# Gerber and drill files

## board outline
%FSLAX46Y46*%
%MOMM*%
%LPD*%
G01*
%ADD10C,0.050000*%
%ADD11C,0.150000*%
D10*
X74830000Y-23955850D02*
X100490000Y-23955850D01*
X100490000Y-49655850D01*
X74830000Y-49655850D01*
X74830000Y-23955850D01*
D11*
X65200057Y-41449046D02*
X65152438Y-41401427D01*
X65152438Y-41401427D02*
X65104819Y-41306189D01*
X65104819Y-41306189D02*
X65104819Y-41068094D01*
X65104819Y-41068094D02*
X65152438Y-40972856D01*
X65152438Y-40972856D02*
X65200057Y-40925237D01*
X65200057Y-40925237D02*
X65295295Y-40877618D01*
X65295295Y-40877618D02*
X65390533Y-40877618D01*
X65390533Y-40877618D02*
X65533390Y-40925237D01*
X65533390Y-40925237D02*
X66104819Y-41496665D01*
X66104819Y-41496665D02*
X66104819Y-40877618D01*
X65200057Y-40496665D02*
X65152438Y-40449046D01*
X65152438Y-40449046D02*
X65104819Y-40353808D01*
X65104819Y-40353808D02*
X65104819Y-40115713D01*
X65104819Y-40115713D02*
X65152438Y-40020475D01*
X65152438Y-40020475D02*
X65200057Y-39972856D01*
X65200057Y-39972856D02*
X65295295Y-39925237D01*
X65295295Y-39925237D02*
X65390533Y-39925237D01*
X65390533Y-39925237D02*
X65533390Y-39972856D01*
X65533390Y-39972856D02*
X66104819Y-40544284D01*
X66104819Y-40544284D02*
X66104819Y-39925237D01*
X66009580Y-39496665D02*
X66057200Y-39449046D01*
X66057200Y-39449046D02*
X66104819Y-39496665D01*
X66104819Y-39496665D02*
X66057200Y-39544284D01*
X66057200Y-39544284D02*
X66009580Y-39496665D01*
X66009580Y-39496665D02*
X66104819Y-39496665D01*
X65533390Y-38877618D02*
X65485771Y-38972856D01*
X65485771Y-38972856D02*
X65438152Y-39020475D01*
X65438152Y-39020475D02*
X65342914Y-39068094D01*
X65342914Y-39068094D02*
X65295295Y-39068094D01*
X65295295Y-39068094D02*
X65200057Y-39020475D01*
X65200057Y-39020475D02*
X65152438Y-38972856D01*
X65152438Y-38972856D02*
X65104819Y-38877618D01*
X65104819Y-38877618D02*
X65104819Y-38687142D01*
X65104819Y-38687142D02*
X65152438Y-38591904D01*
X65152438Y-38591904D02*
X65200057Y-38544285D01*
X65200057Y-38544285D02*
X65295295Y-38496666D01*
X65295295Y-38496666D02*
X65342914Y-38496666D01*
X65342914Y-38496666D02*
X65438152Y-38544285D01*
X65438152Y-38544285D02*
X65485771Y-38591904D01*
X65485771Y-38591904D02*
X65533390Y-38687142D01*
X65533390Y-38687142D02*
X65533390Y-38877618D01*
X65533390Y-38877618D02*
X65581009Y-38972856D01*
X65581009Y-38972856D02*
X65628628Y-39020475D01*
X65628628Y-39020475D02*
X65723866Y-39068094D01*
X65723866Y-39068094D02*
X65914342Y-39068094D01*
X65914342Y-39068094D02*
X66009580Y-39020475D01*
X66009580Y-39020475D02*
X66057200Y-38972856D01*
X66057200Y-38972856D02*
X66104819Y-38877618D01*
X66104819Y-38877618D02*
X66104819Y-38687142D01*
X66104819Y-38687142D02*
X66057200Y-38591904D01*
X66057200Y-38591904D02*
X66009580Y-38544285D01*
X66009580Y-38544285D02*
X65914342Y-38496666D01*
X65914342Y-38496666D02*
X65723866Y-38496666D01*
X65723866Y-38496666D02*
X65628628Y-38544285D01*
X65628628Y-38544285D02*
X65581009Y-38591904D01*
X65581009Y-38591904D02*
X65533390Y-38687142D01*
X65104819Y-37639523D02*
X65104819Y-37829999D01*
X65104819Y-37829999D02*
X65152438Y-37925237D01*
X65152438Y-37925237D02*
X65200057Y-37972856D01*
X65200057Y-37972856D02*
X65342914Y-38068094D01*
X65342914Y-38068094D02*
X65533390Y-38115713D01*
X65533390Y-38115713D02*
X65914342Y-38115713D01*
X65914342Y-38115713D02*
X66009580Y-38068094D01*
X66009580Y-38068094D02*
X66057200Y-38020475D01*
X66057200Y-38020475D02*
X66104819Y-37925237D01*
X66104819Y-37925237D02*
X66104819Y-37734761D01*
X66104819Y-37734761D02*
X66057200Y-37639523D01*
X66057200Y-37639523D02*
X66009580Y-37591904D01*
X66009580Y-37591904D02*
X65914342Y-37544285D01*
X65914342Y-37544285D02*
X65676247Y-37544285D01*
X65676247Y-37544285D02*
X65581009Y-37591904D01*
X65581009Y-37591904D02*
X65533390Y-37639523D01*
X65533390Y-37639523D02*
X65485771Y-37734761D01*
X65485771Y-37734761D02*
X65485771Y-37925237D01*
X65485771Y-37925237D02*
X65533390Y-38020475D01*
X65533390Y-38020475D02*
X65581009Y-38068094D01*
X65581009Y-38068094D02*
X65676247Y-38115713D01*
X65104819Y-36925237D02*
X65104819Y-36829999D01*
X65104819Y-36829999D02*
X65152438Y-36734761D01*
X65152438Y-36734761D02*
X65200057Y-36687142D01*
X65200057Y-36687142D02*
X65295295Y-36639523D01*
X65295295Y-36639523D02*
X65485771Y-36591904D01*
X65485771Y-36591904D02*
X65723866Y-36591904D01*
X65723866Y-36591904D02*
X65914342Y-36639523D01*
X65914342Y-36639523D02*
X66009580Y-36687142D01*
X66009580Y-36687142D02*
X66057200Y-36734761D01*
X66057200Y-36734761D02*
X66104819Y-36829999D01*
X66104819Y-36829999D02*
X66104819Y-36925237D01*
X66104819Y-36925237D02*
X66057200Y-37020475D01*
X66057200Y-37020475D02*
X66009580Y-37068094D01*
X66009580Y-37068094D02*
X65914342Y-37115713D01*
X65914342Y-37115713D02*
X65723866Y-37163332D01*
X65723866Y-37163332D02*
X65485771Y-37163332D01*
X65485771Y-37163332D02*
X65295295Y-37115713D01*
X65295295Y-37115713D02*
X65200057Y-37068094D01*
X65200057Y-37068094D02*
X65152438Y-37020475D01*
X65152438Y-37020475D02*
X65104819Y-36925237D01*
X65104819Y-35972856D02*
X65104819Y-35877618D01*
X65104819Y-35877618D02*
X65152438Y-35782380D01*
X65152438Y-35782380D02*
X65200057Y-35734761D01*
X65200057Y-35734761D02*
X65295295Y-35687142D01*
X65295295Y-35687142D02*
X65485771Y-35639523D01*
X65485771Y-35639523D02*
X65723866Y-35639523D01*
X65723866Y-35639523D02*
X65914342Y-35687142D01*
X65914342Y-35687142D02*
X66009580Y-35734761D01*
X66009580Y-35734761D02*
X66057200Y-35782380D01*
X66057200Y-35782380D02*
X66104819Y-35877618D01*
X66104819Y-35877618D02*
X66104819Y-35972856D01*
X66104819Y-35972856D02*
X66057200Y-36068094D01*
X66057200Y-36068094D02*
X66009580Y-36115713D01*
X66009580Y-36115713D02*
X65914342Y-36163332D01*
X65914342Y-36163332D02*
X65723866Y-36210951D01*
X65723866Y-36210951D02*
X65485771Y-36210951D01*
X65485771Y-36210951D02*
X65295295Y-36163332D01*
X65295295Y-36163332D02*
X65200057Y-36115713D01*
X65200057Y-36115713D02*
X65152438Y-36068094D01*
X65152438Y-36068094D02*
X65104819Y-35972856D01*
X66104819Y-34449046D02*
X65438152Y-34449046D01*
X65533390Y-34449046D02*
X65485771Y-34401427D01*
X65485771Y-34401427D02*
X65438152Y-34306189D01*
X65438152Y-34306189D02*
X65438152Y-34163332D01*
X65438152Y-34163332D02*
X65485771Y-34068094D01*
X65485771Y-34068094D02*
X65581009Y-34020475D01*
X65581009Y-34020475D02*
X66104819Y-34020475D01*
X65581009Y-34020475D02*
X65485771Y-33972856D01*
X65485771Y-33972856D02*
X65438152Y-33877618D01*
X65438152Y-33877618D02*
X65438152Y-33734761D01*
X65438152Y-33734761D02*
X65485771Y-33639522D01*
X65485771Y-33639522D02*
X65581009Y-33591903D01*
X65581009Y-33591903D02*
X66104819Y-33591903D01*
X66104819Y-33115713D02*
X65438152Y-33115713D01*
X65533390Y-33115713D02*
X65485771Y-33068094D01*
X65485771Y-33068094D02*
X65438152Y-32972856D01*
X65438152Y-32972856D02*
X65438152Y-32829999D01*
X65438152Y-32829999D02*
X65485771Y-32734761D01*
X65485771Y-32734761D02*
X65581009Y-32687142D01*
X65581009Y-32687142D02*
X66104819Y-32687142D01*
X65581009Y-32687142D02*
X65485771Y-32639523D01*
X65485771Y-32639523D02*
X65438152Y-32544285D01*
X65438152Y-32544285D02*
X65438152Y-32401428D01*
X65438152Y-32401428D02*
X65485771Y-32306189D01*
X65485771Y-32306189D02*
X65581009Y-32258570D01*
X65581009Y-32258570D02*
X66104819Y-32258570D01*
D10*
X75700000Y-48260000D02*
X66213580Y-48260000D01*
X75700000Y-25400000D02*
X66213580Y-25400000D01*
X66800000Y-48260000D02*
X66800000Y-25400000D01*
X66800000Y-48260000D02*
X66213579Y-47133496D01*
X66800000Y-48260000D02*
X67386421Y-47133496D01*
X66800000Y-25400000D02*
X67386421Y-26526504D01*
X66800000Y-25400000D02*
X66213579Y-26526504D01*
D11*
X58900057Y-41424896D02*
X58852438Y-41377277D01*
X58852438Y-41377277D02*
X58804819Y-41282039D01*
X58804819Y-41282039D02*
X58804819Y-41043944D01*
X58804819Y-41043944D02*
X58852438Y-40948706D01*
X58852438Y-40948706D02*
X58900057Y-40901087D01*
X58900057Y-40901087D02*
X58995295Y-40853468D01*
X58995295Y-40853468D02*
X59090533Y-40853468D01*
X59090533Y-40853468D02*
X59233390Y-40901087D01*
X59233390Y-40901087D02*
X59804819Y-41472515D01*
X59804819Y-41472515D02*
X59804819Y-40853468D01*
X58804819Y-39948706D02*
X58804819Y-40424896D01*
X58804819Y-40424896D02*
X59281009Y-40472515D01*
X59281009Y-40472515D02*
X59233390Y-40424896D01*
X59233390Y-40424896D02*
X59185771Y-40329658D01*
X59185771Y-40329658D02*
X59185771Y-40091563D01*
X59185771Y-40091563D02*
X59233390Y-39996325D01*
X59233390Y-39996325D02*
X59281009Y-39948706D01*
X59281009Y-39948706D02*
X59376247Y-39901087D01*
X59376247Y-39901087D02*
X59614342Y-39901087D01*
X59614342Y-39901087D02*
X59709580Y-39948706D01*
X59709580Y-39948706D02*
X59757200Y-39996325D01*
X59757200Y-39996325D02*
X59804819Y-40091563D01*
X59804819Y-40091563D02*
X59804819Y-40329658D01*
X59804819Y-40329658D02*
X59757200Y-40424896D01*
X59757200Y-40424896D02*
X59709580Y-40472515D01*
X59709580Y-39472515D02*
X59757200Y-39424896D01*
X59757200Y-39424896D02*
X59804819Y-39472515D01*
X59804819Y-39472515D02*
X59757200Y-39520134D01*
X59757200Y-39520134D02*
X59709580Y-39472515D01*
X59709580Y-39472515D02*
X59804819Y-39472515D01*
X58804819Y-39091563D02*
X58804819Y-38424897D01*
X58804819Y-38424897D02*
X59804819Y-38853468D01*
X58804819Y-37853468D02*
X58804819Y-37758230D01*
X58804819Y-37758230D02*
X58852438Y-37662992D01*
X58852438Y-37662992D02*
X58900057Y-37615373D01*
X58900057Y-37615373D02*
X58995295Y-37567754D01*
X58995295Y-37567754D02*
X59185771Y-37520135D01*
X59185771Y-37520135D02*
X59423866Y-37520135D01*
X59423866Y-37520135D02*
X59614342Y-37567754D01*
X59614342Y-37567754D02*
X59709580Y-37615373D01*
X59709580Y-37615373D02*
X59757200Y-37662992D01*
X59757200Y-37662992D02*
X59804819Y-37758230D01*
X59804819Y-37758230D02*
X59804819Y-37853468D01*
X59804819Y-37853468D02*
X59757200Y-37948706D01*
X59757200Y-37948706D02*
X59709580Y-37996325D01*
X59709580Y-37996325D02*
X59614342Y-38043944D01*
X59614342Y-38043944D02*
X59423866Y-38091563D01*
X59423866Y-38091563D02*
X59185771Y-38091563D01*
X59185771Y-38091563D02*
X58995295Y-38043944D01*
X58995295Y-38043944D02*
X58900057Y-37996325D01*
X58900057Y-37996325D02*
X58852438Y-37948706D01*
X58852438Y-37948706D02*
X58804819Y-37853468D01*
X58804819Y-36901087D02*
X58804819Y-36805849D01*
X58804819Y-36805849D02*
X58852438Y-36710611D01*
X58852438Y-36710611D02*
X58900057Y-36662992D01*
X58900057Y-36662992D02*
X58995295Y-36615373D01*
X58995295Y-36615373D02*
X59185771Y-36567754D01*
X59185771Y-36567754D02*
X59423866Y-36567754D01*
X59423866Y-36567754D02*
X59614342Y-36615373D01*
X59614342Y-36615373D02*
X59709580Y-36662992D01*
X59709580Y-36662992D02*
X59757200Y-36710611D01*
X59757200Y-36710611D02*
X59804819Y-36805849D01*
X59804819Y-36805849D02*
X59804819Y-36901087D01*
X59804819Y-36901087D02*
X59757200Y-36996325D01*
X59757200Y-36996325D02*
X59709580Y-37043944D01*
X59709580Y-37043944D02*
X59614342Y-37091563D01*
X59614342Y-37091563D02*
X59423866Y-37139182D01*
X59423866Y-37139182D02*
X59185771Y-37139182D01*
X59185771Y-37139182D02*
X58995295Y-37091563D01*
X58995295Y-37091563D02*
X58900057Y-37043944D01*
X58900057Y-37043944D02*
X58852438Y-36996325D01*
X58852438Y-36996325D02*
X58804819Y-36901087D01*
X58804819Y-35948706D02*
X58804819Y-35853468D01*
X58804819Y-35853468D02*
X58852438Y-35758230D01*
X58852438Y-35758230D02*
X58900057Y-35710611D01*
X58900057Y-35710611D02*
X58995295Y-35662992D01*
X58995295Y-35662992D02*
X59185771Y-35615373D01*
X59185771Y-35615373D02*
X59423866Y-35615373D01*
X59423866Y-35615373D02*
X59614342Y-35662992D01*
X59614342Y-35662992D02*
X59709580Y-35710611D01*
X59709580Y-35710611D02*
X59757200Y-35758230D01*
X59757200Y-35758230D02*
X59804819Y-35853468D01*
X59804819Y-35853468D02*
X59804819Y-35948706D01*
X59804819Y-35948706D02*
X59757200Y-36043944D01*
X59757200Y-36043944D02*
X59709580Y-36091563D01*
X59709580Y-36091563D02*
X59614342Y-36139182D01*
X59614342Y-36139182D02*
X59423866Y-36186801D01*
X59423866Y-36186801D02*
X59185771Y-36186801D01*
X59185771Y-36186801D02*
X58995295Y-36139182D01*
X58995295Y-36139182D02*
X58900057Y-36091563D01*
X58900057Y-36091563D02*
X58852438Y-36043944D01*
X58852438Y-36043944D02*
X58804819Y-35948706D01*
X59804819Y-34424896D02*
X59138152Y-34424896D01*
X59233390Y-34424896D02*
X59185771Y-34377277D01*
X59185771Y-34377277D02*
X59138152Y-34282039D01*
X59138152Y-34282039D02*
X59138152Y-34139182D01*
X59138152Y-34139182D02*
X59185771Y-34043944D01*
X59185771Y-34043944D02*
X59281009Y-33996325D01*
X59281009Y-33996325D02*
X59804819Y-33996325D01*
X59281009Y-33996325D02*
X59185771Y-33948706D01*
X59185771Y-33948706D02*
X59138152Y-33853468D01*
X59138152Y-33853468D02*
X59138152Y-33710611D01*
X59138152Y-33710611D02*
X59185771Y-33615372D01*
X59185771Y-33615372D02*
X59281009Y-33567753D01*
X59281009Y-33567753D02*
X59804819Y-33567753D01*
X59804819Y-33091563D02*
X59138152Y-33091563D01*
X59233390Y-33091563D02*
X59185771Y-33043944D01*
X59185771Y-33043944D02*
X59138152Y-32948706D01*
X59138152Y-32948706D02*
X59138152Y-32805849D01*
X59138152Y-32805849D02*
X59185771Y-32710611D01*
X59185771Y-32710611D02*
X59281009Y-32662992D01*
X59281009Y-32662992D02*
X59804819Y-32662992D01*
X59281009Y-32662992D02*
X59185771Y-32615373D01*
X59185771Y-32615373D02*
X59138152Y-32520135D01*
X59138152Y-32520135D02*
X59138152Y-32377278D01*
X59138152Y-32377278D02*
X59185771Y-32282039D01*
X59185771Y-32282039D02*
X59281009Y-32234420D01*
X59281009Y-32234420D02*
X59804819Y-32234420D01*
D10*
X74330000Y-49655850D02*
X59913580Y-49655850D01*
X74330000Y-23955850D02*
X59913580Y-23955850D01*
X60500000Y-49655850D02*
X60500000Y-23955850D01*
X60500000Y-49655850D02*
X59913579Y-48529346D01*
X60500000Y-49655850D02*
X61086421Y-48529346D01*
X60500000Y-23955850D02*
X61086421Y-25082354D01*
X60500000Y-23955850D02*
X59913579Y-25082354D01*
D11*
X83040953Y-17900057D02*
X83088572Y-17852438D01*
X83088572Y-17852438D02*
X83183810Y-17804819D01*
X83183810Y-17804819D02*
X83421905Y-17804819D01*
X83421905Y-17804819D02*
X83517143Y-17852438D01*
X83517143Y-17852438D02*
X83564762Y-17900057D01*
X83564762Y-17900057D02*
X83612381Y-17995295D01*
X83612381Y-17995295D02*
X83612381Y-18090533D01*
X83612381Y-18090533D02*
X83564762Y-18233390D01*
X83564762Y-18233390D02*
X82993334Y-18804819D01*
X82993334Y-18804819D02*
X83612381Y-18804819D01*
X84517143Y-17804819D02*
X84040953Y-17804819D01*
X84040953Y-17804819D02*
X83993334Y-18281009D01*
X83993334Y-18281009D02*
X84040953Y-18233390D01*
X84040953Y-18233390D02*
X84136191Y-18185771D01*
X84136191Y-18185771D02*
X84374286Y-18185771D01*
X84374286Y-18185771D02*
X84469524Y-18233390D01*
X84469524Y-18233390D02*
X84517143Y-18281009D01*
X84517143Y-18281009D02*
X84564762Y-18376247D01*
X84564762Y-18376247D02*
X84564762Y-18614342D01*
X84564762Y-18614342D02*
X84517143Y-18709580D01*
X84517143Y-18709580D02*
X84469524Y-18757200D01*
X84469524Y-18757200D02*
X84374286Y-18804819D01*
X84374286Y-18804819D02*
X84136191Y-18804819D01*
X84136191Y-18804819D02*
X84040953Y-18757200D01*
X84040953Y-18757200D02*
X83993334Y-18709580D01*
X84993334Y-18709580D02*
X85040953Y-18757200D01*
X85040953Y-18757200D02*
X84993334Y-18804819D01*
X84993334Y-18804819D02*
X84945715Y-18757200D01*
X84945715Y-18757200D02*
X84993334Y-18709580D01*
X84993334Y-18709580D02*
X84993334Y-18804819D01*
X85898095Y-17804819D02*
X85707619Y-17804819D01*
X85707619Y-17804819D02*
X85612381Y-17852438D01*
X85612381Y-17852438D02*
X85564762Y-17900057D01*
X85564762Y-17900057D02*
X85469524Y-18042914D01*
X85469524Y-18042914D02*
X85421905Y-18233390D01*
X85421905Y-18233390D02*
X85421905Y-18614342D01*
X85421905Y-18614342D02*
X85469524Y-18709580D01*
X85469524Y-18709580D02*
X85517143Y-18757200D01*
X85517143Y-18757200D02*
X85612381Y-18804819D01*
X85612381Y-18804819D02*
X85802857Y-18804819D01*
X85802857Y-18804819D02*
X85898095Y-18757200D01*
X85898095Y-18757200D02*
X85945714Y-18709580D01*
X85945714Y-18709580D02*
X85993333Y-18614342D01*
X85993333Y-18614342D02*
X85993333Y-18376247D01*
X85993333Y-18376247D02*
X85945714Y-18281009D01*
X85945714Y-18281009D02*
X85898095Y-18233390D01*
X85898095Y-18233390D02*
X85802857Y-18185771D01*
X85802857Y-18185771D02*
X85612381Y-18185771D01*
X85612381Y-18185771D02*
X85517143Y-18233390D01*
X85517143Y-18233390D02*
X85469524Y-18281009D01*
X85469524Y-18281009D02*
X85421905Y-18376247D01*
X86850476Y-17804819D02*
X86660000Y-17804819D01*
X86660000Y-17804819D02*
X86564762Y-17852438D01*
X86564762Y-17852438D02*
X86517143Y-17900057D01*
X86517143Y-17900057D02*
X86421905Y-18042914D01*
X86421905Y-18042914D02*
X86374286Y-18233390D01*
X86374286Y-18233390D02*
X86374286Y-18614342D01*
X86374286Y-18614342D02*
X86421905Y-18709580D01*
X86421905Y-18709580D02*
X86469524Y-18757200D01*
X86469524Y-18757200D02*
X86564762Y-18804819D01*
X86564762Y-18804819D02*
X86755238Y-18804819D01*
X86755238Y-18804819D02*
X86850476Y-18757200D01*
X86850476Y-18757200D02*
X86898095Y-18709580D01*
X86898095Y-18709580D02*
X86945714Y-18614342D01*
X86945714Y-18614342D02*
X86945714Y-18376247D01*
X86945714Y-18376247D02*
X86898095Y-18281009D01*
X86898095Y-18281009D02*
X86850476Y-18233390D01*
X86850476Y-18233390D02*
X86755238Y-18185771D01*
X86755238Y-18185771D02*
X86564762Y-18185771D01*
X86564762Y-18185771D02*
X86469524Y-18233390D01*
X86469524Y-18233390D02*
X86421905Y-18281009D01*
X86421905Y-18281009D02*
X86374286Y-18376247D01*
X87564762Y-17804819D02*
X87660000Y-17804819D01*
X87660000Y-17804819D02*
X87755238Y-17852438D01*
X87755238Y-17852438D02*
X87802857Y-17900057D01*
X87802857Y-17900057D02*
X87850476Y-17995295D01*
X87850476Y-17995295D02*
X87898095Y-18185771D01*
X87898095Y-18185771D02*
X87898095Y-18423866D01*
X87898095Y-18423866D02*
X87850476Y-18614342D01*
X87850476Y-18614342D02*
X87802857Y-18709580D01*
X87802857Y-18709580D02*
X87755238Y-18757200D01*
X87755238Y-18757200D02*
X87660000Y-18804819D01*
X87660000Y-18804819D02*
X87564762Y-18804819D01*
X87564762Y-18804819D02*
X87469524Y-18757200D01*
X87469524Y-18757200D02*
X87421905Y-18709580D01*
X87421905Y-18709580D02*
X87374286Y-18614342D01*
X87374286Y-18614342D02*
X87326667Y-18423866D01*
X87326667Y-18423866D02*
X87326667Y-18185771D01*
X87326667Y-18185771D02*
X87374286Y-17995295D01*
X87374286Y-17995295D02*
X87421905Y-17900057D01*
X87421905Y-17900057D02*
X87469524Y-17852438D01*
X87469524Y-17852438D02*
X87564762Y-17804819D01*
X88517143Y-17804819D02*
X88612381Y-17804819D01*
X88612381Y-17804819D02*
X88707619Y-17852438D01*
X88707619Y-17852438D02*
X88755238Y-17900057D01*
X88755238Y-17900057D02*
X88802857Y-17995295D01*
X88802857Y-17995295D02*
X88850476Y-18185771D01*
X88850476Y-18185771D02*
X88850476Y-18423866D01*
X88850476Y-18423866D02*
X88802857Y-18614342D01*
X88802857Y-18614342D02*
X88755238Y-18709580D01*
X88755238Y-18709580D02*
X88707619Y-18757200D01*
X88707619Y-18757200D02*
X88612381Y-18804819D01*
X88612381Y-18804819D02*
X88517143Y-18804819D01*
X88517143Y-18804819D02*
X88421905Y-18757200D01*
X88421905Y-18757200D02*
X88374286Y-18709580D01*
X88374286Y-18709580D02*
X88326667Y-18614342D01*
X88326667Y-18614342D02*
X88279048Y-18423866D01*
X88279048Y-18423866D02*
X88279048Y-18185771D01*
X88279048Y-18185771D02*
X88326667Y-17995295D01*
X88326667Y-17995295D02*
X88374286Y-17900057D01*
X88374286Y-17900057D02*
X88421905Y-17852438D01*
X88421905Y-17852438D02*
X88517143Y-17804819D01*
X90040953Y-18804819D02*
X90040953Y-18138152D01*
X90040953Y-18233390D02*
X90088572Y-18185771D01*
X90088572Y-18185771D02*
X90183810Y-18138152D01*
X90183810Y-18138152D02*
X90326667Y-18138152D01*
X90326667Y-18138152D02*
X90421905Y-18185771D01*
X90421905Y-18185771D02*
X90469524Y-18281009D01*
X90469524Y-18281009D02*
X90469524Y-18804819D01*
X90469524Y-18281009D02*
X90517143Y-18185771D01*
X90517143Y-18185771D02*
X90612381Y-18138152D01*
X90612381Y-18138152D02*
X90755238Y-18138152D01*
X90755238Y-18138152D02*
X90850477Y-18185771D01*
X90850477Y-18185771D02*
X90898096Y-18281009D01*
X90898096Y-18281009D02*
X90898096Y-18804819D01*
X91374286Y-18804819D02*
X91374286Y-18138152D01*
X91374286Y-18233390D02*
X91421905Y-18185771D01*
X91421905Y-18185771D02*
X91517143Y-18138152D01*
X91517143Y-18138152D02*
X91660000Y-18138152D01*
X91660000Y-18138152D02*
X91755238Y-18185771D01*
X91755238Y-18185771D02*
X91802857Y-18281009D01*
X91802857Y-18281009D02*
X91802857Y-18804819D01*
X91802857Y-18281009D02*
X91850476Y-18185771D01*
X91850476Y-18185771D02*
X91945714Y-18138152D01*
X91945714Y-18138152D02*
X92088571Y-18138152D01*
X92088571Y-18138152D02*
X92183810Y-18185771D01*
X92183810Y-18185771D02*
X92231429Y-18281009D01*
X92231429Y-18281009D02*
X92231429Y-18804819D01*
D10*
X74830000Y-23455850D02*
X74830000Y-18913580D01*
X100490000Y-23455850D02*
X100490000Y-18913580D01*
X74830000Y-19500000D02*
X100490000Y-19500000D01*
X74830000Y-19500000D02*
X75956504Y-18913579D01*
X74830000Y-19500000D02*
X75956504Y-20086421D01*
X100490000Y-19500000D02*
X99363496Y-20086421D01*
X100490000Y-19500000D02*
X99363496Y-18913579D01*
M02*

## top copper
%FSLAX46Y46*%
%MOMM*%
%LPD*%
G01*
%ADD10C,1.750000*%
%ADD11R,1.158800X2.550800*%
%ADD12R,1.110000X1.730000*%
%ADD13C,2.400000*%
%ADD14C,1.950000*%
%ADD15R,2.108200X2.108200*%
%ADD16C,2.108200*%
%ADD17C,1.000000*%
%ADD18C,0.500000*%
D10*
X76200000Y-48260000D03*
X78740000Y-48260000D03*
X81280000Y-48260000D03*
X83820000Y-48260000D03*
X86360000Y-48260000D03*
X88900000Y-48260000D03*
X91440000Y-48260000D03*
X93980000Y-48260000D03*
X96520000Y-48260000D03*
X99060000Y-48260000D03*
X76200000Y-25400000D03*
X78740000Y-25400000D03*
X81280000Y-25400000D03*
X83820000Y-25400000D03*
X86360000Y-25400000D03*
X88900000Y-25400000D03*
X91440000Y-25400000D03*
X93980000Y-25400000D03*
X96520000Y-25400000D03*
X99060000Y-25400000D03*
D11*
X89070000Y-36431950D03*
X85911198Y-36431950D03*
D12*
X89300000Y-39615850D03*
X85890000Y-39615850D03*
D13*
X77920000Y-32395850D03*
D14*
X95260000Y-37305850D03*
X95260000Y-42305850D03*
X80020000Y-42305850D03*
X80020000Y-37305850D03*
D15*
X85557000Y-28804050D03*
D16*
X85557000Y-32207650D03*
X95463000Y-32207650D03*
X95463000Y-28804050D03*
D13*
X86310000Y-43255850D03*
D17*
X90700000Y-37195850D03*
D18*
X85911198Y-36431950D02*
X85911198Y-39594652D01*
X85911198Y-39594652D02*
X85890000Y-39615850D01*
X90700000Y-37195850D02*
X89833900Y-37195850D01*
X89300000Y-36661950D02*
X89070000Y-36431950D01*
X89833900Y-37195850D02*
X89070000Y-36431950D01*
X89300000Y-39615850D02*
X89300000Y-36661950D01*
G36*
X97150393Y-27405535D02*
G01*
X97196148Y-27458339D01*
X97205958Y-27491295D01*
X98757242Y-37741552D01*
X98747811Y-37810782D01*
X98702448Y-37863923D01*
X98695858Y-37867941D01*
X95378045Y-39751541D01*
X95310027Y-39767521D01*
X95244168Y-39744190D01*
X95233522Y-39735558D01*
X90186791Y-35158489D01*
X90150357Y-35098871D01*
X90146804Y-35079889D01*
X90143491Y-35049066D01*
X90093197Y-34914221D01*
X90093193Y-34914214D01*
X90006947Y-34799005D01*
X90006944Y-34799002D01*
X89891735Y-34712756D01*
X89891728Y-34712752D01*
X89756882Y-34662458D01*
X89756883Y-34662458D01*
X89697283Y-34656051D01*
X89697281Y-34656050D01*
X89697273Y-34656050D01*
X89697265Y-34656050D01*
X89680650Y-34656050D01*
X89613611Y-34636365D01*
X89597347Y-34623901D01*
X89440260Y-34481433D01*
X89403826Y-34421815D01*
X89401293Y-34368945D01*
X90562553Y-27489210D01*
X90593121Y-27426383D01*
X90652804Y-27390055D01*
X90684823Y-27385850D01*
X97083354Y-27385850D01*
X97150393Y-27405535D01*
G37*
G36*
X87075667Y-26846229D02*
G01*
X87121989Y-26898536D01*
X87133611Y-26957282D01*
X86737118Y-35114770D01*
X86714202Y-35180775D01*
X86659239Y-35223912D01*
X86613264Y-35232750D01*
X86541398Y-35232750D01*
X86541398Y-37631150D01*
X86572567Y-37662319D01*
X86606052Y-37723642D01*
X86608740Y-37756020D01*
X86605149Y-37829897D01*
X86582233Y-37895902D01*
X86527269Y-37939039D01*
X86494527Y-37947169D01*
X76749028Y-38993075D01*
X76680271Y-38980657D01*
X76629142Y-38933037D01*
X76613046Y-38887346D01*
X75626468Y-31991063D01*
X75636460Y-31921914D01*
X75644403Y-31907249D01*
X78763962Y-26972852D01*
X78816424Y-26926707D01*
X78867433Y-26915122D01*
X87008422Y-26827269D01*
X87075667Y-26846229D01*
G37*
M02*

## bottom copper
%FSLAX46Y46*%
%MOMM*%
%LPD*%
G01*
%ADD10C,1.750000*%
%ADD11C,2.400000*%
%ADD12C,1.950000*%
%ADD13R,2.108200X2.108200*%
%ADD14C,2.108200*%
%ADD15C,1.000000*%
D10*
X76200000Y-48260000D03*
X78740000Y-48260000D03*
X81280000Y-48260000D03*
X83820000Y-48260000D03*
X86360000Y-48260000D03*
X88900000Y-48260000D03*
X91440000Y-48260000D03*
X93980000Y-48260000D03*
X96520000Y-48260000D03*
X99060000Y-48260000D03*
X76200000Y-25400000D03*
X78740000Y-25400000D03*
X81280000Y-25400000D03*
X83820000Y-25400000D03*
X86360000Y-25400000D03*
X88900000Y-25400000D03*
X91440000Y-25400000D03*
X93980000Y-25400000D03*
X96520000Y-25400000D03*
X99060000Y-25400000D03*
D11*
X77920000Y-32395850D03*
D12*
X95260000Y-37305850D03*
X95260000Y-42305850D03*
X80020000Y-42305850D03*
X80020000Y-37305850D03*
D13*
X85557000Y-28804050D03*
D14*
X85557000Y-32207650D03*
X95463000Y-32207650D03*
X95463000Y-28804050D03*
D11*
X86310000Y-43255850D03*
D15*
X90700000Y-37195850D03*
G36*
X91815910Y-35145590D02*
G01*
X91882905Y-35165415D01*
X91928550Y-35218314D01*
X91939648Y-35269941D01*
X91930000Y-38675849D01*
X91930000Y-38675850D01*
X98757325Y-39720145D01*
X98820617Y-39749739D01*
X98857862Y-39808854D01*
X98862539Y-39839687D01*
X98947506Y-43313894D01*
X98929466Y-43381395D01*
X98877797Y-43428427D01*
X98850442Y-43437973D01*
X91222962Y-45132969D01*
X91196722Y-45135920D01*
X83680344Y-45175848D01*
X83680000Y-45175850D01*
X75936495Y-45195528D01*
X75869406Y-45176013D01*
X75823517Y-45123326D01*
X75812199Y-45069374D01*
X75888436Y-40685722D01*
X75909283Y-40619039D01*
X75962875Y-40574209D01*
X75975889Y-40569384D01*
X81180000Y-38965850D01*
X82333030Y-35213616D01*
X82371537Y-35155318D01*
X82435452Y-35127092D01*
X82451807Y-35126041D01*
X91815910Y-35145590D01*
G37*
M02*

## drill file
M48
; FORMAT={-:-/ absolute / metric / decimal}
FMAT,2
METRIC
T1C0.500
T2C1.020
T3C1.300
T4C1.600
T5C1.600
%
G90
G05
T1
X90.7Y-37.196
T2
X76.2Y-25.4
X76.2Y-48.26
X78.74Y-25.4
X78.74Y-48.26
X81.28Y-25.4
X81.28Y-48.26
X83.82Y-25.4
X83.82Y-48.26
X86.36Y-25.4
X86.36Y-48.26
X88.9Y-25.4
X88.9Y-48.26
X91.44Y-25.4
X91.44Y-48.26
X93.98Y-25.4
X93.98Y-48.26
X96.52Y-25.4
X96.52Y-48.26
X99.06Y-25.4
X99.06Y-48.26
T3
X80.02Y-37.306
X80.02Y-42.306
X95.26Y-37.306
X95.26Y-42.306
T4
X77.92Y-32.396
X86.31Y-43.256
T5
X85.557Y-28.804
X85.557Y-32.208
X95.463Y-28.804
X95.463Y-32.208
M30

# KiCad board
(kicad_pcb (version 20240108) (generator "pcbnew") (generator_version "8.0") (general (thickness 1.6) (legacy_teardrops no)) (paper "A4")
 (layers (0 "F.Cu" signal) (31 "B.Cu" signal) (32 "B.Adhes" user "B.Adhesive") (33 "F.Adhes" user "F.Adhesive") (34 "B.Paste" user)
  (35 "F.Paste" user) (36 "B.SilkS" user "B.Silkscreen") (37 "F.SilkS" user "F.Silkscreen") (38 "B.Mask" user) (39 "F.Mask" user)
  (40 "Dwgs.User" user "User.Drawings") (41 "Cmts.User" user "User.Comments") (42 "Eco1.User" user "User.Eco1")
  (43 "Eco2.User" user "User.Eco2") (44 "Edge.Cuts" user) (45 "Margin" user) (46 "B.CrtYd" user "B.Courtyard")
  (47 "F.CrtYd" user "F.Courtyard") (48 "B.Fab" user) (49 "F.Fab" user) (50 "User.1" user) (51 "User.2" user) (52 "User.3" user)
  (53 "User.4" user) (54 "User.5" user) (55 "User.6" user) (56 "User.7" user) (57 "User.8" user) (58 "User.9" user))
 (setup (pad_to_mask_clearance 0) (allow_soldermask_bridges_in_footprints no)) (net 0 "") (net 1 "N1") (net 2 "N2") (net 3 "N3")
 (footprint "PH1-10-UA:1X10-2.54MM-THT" (layer "F.Cu") (at 76.2 48.26)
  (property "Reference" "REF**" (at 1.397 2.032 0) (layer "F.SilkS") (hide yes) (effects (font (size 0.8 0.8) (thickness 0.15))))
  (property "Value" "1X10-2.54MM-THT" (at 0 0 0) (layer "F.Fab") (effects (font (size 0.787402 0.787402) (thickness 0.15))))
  (pad "1" thru_hole circle (at 0 0) (size 1.75 1.75) (drill 1.02) (layers "*.Cu" "*.Mask") (remove_unused_layers no)
   (solder_mask_margin 0.102))
  (pad "2" thru_hole circle (at 2.54 0) (size 1.75 1.75) (drill 1.02) (layers "*.Cu" "*.Mask") (remove_unused_layers no)
   (solder_mask_margin 0.102))
  (pad "3" thru_hole circle (at 5.08 0) (size 1.75 1.75) (drill 1.02) (layers "*.Cu" "*.Mask") (remove_unused_layers no)
   (solder_mask_margin 0.102))
  (pad "4" thru_hole circle (at 7.62 0) (size 1.75 1.75) (drill 1.02) (layers "*.Cu" "*.Mask") (remove_unused_layers no)
   (solder_mask_margin 0.102))
  (pad "5" thru_hole circle (at 10.16 0) (size 1.75 1.75) (drill 1.02) (layers "*.Cu" "*.Mask") (remove_unused_layers no)
   (solder_mask_margin 0.102))
  (pad "6" thru_hole circle (at 12.7 0) (size 1.75 1.75) (drill 1.02) (layers "*.Cu" "*.Mask") (remove_unused_layers no)
   (solder_mask_margin 0.102))
  (pad "7" thru_hole circle (at 15.24 0) (size 1.75 1.75) (drill 1.02) (layers "*.Cu" "*.Mask") (remove_unused_layers no)
   (solder_mask_margin 0.102))
  (pad "8" thru_hole circle (at 17.78 0) (size 1.75 1.75) (drill 1.02) (layers "*.Cu" "*.Mask") (remove_unused_layers no)
   (solder_mask_margin 0.102))
  (pad "9" thru_hole circle (at 20.32 0) (size 1.75 1.75) (drill 1.02) (layers "*.Cu" "*.Mask") (remove_unused_layers no)
   (solder_mask_margin 0.102))
  (pad "10" thru_hole circle (at 22.86 0) (size 1.75 1.75) (drill 1.02) (layers "*.Cu" "*.Mask") (remove_unused_layers no)
   (solder_mask_margin 0.102)))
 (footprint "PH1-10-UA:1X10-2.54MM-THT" (layer "F.Cu") (at 76.2 25.4)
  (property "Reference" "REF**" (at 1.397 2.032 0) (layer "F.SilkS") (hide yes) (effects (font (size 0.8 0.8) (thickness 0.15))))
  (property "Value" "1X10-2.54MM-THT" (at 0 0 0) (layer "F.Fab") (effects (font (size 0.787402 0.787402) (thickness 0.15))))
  (pad "1" thru_hole circle (at 0 0) (size 1.75 1.75) (drill 1.02) (layers "*.Cu" "*.Mask") (remove_unused_layers no)
   (solder_mask_margin 0.102))
  (pad "2" thru_hole circle (at 2.54 0) (size 1.75 1.75) (drill 1.02) (layers "*.Cu" "*.Mask") (remove_unused_layers no)
   (solder_mask_margin 0.102))
  (pad "3" thru_hole circle (at 5.08 0) (size 1.75 1.75) (drill 1.02) (layers "*.Cu" "*.Mask") (remove_unused_layers no)
   (solder_mask_margin 0.102))
  (pad "4" thru_hole circle (at 7.62 0) (size 1.75 1.75) (drill 1.02) (layers "*.Cu" "*.Mask") (remove_unused_layers no)
   (solder_mask_margin 0.102))
  (pad "5" thru_hole circle (at 10.16 0) (size 1.75 1.75) (drill 1.02) (layers "*.Cu" "*.Mask") (remove_unused_layers no)
   (solder_mask_margin 0.102))
  (pad "6" thru_hole circle (at 12.7 0) (size 1.75 1.75) (drill 1.02) (layers "*.Cu" "*.Mask") (remove_unused_layers no)
   (solder_mask_margin 0.102))
  (pad "7" thru_hole circle (at 15.24 0) (size 1.75 1.75) (drill 1.02) (layers "*.Cu" "*.Mask") (remove_unused_layers no)
   (solder_mask_margin 0.102))
  (pad "8" thru_hole circle (at 17.78 0) (size 1.75 1.75) (drill 1.02) (layers "*.Cu" "*.Mask") (remove_unused_layers no)
   (solder_mask_margin 0.102))
  (pad "9" thru_hole circle (at 20.32 0) (size 1.75 1.75) (drill 1.02) (layers "*.Cu" "*.Mask") (remove_unused_layers no)
   (solder_mask_margin 0.102))
  (pad "10" thru_hole circle (at 22.86 0) (size 1.75 1.75) (drill 1.02) (layers "*.Cu" "*.Mask") (remove_unused_layers no)
   (solder_mask_margin 0.102)))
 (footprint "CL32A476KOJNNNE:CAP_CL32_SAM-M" (layer "F.Cu") (at 87.490599 36.43195 180)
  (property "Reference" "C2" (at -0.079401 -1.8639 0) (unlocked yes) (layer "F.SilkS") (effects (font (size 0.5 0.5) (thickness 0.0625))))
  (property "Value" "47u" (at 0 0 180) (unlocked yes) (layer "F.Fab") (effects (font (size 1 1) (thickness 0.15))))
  (pad "1" smd rect (at -1.579401 0 180) (size 1.1588 2.5508) (layers "F.Cu" "F.Paste" "F.Mask") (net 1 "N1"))
  (pad "2" smd rect (at 1.579401 0 180) (size 1.1588 2.5508) (layers "F.Cu" "F.Paste" "F.Mask") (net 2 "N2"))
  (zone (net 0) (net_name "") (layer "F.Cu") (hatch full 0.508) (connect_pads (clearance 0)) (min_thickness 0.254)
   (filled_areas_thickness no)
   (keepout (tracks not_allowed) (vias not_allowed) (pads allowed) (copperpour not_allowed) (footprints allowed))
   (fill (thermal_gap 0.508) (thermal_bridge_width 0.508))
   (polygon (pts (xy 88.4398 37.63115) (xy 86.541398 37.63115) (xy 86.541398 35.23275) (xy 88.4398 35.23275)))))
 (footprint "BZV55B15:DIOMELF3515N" (layer "F.Cu") (at 87.595 39.61585)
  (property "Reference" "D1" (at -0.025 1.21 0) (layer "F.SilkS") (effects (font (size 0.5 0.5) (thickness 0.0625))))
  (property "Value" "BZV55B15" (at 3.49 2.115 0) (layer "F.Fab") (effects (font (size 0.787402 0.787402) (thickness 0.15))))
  (pad "A" smd rect (at 1.705 0) (size 1.11 1.73) (layers "F.Cu" "F.Paste" "F.Mask") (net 1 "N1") (solder_mask_margin 0.102))
  (pad "C" smd rect (at -1.705 0) (size 1.11 1.73) (layers "F.Cu" "F.Paste" "F.Mask") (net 2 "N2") (solder_mask_margin 0.102)))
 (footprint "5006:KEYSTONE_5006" (layer "F.Cu") (at 77.92 32.39585)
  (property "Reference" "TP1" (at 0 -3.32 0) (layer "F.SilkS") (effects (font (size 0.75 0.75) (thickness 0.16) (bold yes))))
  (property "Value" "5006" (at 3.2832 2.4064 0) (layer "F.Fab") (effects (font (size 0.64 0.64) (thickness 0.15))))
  (pad "TP" thru_hole circle (at 0 0) (size 2.4 2.4) (drill 1.6) (layers "*.Cu" "*.Mask") (remove_unused_layers no) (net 2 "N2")
   (solder_mask_margin 0.102)))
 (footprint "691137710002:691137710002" (layer "F.Cu") (at 95.26 39.80585 -90)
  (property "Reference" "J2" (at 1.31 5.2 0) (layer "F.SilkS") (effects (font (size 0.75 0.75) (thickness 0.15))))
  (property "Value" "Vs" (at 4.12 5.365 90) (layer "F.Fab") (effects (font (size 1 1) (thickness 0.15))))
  (pad "1" thru_hole circle (at -2.5 0 270) (size 1.95 1.95) (drill 1.3) (layers "*.Cu" "*.Mask") (remove_unused_layers no) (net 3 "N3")
   (solder_mask_margin 0.102))
  (pad "2" thru_hole circle (at 2.5 0 270) (size 1.95 1.95) (drill 1.3) (layers "*.Cu" "*.Mask") (remove_unused_layers no) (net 1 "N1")
   (solder_mask_margin 0.102)))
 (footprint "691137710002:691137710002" (layer "F.Cu") (at 80.02 39.80585 90)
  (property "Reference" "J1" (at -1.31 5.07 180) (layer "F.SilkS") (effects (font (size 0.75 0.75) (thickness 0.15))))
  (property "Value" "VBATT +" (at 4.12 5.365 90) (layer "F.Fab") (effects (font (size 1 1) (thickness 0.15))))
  (pad "1" thru_hole circle (at -2.5 0 90) (size 1.95 1.95) (drill 1.3) (layers "*.Cu" "*.Mask") (remove_unused_layers no) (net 1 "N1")
   (solder_mask_margin 0.102))
  (pad "2" thru_hole circle (at 2.5 0 90) (size 1.95 1.95) (drill 1.3) (layers "*.Cu" "*.Mask") (remove_unused_layers no) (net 2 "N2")
   (solder_mask_margin 0.102)))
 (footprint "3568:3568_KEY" (layer "F.Cu") (at 85.557 28.80405)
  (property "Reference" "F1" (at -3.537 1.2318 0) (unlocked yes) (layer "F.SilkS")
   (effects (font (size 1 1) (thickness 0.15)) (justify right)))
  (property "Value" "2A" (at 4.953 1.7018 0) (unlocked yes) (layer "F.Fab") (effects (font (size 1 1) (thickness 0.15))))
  (pad "1" thru_hole rect (at 0 0) (size 2.1082 2.1082) (drill 1.6002) (layers "*.Cu" "*.Mask") (remove_unused_layers no) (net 2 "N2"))
  (pad "2" thru_hole circle (at 0 3.4036) (size 2.1082 2.1082) (drill 1.6002) (layers "*.Cu" "*.Mask") (remove_unused_layers no)
   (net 2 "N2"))
  (pad "3" thru_hole circle (at 9.906 3.4036) (size 2.1082 2.1082) (drill 1.6002) (layers "*.Cu" "*.Mask") (remove_unused_layers no)
   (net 3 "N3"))
  (pad "4" thru_hole circle (at 9.906 0) (size 2.1082 2.1082) (drill 1.6002) (layers "*.Cu" "*.Mask") (remove_unused_layers no) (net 3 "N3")))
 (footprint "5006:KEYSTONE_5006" (layer "F.Cu") (at 86.31 43.25585)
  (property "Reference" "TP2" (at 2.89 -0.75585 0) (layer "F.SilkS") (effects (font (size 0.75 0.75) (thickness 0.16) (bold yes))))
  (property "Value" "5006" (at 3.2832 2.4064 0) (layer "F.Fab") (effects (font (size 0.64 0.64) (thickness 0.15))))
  (pad "TP" thru_hole circle (at 0 0) (size 2.4 2.4) (drill 1.6) (layers "*.Cu" "*.Mask") (remove_unused_layers no) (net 1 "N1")
   (solder_mask_margin 0.102)))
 (gr_rect (start 74.83 23.95585) (end 100.49 49.65585) (stroke (width 0.05) (type default)) (fill none) (layer "Edge.Cuts"))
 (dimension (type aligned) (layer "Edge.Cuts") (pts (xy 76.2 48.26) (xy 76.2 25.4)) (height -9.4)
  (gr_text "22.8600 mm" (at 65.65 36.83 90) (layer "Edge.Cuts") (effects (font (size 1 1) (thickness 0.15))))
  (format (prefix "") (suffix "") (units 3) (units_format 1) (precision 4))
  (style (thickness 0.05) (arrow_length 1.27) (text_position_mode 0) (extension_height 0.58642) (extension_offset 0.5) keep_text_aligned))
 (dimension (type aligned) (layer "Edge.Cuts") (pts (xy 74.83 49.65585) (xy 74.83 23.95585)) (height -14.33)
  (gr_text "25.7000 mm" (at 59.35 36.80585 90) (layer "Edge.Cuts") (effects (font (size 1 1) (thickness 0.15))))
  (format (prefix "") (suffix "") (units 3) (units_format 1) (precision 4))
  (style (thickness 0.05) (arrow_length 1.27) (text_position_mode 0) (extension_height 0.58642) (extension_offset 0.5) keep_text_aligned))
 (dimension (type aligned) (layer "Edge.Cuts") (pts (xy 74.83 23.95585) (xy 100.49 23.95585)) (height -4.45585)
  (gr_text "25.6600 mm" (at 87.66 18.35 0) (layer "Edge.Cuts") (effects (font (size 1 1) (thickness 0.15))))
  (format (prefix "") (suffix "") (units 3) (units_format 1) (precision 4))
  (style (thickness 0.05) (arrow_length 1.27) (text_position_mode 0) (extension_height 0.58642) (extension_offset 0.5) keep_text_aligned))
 (segment (start 85.911198 36.43195) (end 85.911198 39.594652) (width 0.5) (layer "F.Cu") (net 2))
 (segment (start 85.911198 39.594652) (end 85.89 39.61585) (width 0.5) (layer "F.Cu") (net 2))
 (segment (start 90.7 37.19585) (end 89.8339 37.19585) (width 0.5) (layer "F.Cu") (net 1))
 (segment (start 89.3 36.66195) (end 89.07 36.43195) (width 0.5) (layer "F.Cu") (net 1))
 (segment (start 89.8339 37.19585) (end 89.07 36.43195) (width 0.5) (layer "F.Cu") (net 1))
 (segment (start 89.3 39.61585) (end 89.3 36.66195) (width 0.5) (layer "F.Cu") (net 1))
 (via (at 90.7 37.19585) (size 1) (drill 0.5) (layers "F.Cu" "B.Cu") (free yes) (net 1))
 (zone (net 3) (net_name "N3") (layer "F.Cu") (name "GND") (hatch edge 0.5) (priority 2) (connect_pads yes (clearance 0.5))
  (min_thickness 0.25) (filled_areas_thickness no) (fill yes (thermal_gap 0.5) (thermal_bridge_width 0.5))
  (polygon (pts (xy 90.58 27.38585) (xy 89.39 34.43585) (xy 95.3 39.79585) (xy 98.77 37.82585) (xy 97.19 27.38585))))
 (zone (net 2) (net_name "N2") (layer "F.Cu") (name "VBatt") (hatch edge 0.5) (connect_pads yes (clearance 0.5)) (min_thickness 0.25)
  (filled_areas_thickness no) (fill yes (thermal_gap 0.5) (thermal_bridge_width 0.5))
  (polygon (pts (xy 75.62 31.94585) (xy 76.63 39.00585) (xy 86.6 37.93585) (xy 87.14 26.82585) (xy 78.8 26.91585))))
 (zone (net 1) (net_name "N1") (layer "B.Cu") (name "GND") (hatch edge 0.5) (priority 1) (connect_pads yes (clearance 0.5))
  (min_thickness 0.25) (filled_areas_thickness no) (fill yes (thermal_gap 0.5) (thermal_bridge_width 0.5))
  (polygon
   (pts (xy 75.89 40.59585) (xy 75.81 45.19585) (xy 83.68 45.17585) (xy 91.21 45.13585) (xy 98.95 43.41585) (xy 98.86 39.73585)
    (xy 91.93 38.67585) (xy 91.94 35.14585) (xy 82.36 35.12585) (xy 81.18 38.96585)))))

